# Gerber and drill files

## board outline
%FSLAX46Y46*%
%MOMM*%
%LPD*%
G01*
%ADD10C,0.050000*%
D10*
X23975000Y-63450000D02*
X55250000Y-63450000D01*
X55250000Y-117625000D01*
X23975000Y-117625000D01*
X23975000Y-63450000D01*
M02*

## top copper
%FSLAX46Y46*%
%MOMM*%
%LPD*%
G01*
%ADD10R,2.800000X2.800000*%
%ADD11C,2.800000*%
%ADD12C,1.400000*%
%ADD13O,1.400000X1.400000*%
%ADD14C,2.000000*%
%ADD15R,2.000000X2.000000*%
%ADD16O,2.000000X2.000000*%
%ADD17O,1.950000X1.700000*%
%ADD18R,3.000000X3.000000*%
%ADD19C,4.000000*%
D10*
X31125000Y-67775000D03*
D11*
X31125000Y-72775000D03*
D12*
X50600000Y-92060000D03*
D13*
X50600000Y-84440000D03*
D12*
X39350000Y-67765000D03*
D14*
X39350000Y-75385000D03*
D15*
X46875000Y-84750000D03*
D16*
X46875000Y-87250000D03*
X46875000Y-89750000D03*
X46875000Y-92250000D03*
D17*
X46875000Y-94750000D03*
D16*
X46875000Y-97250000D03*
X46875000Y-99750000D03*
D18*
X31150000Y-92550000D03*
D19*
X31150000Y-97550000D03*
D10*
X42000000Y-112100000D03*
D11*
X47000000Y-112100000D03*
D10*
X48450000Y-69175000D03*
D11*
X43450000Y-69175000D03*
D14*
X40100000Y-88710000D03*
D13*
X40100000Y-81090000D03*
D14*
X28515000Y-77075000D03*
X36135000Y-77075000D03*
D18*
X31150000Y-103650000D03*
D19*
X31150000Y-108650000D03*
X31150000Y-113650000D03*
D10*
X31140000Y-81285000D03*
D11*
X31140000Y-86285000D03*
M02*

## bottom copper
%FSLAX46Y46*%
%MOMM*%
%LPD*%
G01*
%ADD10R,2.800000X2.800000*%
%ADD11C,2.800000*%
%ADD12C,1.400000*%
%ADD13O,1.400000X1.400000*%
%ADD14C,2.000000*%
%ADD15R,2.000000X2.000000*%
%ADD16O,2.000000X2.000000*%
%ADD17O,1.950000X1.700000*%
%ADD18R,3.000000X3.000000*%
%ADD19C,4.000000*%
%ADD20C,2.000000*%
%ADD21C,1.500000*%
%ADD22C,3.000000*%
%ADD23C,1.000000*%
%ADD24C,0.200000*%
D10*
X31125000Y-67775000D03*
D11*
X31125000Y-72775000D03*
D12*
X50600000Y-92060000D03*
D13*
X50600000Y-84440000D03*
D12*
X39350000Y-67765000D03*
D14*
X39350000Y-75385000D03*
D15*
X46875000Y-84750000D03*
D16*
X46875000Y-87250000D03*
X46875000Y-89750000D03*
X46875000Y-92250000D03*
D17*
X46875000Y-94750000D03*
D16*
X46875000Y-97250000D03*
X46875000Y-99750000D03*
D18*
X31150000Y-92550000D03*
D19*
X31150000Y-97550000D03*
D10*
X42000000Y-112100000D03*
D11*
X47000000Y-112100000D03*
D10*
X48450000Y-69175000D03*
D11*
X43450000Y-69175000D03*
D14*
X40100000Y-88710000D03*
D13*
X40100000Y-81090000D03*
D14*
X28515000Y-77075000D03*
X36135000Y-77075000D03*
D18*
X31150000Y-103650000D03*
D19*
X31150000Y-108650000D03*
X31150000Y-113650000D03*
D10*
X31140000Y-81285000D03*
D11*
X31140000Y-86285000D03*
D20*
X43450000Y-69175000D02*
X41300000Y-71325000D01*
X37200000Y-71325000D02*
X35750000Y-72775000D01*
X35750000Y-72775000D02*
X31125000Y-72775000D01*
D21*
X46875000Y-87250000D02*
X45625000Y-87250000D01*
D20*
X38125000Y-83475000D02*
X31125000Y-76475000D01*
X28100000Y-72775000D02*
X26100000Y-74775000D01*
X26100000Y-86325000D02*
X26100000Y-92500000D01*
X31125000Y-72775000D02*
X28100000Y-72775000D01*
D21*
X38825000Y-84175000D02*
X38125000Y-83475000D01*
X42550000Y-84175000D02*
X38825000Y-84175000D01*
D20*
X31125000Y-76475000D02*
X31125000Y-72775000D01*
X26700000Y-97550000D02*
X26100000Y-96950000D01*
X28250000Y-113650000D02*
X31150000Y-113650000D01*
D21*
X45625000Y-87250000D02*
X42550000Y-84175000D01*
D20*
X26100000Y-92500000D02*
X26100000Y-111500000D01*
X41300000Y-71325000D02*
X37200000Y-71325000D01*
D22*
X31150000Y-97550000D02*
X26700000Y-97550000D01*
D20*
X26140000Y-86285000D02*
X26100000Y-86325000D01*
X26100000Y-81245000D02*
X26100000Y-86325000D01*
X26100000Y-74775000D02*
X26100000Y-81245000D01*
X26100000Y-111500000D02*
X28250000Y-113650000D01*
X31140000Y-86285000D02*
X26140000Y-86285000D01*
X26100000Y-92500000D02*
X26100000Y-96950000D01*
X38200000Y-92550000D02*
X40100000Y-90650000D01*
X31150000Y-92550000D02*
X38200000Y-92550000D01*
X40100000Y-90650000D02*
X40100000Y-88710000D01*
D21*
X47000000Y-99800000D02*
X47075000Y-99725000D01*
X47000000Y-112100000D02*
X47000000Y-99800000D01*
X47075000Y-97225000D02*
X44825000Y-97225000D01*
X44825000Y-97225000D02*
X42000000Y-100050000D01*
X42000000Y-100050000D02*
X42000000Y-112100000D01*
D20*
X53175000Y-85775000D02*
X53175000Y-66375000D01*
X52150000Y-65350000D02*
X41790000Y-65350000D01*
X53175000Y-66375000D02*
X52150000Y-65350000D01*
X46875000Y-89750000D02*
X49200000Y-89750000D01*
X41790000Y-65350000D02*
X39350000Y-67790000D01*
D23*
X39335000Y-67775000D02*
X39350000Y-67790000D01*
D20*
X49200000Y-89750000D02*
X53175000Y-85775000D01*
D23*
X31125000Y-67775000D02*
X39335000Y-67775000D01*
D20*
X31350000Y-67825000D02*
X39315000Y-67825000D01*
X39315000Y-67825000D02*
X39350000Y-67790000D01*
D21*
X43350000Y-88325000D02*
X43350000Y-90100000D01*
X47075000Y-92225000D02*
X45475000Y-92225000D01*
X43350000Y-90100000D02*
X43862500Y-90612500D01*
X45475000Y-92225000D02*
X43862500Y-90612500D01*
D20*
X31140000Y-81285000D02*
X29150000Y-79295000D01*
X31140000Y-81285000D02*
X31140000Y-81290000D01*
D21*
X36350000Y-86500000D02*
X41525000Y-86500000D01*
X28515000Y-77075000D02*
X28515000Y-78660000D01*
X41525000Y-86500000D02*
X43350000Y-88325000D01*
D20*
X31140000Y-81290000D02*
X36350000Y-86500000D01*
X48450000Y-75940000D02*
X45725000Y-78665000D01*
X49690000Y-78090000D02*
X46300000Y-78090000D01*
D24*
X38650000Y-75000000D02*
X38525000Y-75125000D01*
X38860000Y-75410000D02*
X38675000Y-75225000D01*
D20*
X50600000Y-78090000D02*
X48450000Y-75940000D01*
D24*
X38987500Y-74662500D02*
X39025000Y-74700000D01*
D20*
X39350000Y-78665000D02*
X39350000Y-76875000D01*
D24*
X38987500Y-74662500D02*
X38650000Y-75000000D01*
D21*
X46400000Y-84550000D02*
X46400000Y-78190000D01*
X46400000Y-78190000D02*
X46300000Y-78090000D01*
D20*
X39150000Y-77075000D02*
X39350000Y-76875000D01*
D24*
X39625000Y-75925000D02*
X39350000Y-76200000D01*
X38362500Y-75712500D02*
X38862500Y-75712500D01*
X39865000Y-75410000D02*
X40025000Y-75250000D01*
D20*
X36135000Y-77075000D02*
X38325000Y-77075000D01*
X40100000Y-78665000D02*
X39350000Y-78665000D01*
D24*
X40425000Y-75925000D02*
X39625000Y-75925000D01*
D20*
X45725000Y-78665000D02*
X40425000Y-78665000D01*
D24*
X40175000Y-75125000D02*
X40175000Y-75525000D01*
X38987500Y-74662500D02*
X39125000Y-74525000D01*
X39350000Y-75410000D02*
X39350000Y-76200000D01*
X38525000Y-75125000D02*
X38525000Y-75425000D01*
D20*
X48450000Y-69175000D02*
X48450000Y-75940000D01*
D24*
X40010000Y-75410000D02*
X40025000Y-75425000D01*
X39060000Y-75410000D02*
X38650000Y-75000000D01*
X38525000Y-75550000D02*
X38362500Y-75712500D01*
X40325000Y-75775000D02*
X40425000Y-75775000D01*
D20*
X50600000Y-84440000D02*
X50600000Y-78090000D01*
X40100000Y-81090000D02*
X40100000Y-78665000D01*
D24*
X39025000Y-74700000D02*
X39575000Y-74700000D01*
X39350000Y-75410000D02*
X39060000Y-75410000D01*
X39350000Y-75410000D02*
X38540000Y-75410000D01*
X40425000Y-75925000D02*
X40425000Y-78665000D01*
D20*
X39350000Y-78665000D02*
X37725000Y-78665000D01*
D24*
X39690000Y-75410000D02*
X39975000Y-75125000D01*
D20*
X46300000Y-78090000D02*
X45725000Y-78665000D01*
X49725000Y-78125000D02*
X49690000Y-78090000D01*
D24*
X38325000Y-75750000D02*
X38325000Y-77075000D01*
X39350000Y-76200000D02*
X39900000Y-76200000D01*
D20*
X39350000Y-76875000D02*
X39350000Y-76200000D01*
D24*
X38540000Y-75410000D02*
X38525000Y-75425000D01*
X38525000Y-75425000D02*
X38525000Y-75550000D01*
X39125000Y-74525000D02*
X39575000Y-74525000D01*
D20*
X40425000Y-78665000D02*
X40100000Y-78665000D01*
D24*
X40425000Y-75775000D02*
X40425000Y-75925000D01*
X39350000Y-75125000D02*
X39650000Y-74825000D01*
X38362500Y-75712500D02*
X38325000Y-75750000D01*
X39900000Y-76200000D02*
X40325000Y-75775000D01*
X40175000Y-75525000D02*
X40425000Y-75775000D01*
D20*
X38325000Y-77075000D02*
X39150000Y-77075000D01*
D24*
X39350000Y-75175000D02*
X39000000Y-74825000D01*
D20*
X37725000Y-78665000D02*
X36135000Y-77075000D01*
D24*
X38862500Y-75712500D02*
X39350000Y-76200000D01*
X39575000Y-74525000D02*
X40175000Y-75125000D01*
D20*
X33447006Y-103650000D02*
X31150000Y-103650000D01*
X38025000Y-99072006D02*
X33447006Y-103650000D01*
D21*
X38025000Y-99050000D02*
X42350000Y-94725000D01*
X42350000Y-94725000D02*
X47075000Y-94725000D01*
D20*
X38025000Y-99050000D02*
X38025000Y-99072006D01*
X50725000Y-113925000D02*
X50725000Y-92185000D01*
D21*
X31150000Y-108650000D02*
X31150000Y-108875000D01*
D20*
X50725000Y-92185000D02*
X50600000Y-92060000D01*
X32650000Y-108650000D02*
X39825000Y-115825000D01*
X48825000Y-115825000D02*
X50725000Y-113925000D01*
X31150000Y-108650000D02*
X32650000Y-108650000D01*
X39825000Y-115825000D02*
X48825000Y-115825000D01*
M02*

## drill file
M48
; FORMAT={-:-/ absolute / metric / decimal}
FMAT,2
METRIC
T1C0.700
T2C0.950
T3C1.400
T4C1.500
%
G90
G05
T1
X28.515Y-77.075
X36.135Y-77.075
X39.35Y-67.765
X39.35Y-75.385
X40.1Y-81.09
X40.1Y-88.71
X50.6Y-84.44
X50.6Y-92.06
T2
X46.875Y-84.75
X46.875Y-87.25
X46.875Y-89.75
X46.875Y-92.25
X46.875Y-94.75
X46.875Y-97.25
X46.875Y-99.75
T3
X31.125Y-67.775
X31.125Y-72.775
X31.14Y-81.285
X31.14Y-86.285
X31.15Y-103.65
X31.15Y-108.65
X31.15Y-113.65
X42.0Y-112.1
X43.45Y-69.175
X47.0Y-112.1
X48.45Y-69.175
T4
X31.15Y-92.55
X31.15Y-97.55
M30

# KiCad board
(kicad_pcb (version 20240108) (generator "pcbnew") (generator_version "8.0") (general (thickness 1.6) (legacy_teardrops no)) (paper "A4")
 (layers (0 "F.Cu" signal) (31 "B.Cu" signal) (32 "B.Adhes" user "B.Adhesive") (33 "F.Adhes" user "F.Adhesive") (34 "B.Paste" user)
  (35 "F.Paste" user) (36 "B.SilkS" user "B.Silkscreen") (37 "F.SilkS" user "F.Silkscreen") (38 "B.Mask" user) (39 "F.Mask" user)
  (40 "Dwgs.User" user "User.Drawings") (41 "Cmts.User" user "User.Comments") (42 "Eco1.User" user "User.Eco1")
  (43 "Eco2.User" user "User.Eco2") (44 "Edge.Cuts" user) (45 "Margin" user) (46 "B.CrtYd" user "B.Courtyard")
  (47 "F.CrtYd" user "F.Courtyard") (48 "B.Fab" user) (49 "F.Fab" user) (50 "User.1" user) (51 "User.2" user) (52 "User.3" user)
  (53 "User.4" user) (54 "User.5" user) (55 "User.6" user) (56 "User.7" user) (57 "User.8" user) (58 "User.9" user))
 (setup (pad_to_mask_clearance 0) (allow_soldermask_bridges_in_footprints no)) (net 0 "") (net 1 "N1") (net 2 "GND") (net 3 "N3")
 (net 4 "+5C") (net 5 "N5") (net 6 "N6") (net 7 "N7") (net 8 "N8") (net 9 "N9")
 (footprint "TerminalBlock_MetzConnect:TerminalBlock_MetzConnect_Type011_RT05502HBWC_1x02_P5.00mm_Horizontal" (layer "F.Cu")
  (at 31.125 67.775 -90)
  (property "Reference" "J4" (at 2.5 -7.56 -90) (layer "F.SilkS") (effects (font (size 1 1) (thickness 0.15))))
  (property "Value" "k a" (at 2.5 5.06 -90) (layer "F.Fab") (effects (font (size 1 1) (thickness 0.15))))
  (pad "1" thru_hole rect (at 0 0 270) (size 2.8 2.8) (drill 1.4) (layers "*.Cu" "*.Mask") (remove_unused_layers no) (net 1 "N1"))
  (pad "2" thru_hole circle (at 5 0 270) (size 2.8 2.8) (drill 1.4) (layers "*.Cu" "*.Mask") (remove_unused_layers no) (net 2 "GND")))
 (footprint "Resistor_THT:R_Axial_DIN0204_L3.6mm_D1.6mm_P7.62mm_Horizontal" (layer "F.Cu") (at 50.6 92.06 90)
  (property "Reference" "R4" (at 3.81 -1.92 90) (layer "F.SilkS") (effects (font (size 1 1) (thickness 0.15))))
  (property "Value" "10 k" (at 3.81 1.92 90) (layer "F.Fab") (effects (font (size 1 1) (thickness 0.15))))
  (pad "1" thru_hole circle (at 0 0 90) (size 1.4 1.4) (drill 0.7) (layers "*.Cu" "*.Mask") (remove_unused_layers no) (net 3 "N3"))
  (pad "2" thru_hole oval (at 7.62 0 90) (size 1.4 1.4) (drill 0.7) (layers "*.Cu" "*.Mask") (remove_unused_layers no) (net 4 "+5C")))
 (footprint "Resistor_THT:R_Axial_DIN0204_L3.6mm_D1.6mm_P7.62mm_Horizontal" (layer "F.Cu") (at 39.35 67.765 -90)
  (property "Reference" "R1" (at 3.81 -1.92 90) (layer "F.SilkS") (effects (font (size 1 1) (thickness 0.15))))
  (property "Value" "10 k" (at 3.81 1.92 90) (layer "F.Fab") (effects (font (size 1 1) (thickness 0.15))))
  (pad "1" thru_hole circle (at 0 0 270) (size 1.4 1.4) (drill 0.7) (layers "*.Cu" "*.Mask") (remove_unused_layers no) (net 1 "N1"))
  (pad "2" thru_hole circle (at 7.62 0 270) (size 2 2) (drill 0.7) (layers "*.Cu" "*.Mask") (remove_unused_layers no) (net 4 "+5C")))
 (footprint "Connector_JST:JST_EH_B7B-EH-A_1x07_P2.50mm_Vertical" (layer "F.Cu") (at 46.875 84.75 -90)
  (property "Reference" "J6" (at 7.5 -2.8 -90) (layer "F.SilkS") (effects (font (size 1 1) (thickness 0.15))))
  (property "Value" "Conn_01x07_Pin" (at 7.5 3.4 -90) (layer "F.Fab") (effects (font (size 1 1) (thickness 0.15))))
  (pad "1" thru_hole rect (at 0 0 270) (size 2 2) (drill 0.95) (layers "*.Cu" "*.Mask") (remove_unused_layers no) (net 4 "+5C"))
  (pad "2" thru_hole oval (at 2.5 0 270) (size 2 2) (drill 0.95) (layers "*.Cu" "*.Mask") (remove_unused_layers no) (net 2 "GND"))
  (pad "3" thru_hole oval (at 5 0 270) (size 2 2) (drill 0.95) (layers "*.Cu" "*.Mask") (remove_unused_layers no) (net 1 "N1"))
  (pad "4" thru_hole oval (at 7.5 0 270) (size 2 2) (drill 0.95) (layers "*.Cu" "*.Mask") (remove_unused_layers no) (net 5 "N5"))
  (pad "5" thru_hole oval (at 10 0 270) (size 1.7 1.95) (drill 0.95) (layers "*.Cu" "*.Mask") (remove_unused_layers no) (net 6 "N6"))
  (pad "6" thru_hole oval (at 12.5 0 270) (size 2 2) (drill 0.95) (layers "*.Cu" "*.Mask") (remove_unused_layers no) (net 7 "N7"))
  (pad "7" thru_hole oval (at 15 0 270) (size 2 2) (drill 0.95) (layers "*.Cu" "*.Mask") (remove_unused_layers no) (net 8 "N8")))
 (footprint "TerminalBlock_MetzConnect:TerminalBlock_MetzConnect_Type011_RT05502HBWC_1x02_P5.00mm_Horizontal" (layer "F.Cu")
  (at 31.15 92.55 -90)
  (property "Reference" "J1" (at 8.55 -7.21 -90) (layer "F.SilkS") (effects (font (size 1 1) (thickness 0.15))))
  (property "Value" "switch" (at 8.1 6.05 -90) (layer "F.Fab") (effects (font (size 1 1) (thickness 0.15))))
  (pad "1" thru_hole rect (at 0 0 270) (size 3 3) (drill 1.5) (layers "*.Cu" "*.Mask") (remove_unused_layers no) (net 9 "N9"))
  (pad "2" thru_hole circle (at 5 0 270) (size 4 4) (drill 1.5) (layers "*.Cu" "*.Mask") (remove_unused_layers no) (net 2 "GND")))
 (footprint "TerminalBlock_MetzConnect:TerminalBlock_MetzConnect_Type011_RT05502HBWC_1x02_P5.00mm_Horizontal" (layer "F.Cu") (at 42 112.1)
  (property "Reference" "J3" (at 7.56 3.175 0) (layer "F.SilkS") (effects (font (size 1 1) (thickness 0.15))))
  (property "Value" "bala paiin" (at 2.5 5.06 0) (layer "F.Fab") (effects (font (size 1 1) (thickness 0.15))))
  (pad "1" thru_hole rect (at 0 0) (size 2.8 2.8) (drill 1.4) (layers "*.Cu" "*.Mask") (remove_unused_layers no) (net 7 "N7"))
  (pad "2" thru_hole circle (at 5 0) (size 2.8 2.8) (drill 1.4) (layers "*.Cu" "*.Mask") (remove_unused_layers no) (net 8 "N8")))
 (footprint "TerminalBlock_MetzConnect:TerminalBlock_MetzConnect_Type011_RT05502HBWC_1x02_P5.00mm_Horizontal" (layer "F.Cu")
  (at 48.45 69.175 180)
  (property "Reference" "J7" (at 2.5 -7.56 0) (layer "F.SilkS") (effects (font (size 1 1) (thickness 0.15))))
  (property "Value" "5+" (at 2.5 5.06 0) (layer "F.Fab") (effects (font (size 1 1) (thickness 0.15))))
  (pad "1" thru_hole rect (at 0 0 180) (size 2.8 2.8) (drill 1.4) (layers "*.Cu" "*.Mask") (remove_unused_layers no) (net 4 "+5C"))
  (pad "2" thru_hole circle (at 5 0 180) (size 2.8 2.8) (drill 1.4) (layers "*.Cu" "*.Mask") (remove_unused_layers no) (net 2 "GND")))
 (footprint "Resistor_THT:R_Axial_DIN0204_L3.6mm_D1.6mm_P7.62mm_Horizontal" (layer "F.Cu") (at 40.1 88.71 90)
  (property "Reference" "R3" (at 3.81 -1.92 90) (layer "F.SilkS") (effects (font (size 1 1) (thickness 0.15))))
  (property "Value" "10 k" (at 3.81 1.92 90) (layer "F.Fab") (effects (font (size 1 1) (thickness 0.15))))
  (pad "1" thru_hole circle (at 0 0 90) (size 2 2) (drill 0.7) (layers "*.Cu" "*.Mask") (remove_unused_layers no) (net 9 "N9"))
  (pad "2" thru_hole oval (at 7.62 0 90) (size 1.4 1.4) (drill 0.7) (layers "*.Cu" "*.Mask") (remove_unused_layers no) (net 4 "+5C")))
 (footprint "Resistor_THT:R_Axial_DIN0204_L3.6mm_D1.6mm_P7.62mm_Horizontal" (layer "F.Cu") (at 28.515 77.075)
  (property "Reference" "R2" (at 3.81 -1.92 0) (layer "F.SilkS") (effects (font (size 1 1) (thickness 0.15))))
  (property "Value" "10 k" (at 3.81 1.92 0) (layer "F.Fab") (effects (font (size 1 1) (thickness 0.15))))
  (pad "1" thru_hole circle (at 0 0) (size 2 2) (drill 0.7) (layers "*.Cu" "*.Mask") (remove_unused_layers no) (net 5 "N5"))
  (pad "2" thru_hole circle (at 7.62 0) (size 2 2) (drill 0.7) (layers "*.Cu" "*.Mask") (remove_unused_layers no) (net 4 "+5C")))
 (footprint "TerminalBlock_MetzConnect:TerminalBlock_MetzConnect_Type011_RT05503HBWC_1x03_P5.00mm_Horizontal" (layer "F.Cu")
  (at 31.15 103.65 -90)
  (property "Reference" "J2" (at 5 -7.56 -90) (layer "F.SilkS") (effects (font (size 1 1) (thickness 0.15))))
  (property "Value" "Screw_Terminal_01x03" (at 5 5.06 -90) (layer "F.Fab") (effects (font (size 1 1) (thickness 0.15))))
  (pad "1" thru_hole rect (at 0 0 270) (size 3 3) (drill 1.4) (layers "*.Cu" "*.Mask") (remove_unused_layers no) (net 6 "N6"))
  (pad "2" thru_hole circle (at 5 0 270) (size 4 4) (drill 1.4) (layers "*.Cu" "*.Mask") (remove_unused_layers no) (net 3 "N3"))
  (pad "3" thru_hole circle (at 10 0 270) (size 4 4) (drill 1.4) (layers "*.Cu" "*.Mask") (remove_unused_layers no) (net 2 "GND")))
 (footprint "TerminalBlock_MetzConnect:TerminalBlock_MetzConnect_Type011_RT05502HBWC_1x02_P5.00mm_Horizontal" (layer "F.Cu")
  (at 31.14 81.285 -90)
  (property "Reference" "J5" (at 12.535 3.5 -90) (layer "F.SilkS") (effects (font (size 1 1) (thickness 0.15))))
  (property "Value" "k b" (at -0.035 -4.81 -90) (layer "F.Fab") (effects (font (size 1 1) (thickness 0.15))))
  (pad "1" thru_hole rect (at 0 0 270) (size 2.8 2.8) (drill 1.4) (layers "*.Cu" "*.Mask") (remove_unused_layers no) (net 5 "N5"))
  (pad "2" thru_hole circle (at 5 0 270) (size 2.8 2.8) (drill 1.4) (layers "*.Cu" "*.Mask") (remove_unused_layers no) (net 2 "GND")))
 (gr_rect (start 23.975 63.45) (end 55.25 117.625) (stroke (width 0.05) (type default)) (fill none) (layer "Edge.Cuts"))
 (segment (start 43.45 69.175) (end 41.3 71.325) (width 2) (layer "B.Cu") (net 2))
 (segment (start 37.2 71.325) (end 35.75 72.775) (width 2) (layer "B.Cu") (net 2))
 (segment (start 35.75 72.775) (end 31.125 72.775) (width 2) (layer "B.Cu") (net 2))
 (segment (start 46.875 87.25) (end 45.625 87.25) (width 1.5) (layer "B.Cu") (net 2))
 (segment (start 38.125 83.475) (end 31.125 76.475) (width 2) (layer "B.Cu") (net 2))
 (segment (start 28.1 72.775) (end 26.1 74.775) (width 2) (layer "B.Cu") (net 2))
 (segment (start 26.1 86.325) (end 26.1 92.5) (width 2) (layer "B.Cu") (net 2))
 (segment (start 31.125 72.775) (end 28.1 72.775) (width 2) (layer "B.Cu") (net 2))
 (segment (start 38.825 84.175) (end 38.125 83.475) (width 1.5) (layer "B.Cu") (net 2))
 (segment (start 42.55 84.175) (end 38.825 84.175) (width 1.5) (layer "B.Cu") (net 2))
 (segment (start 31.125 76.475) (end 31.125 72.775) (width 2) (layer "B.Cu") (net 2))
 (segment (start 26.7 97.55) (end 26.1 96.95) (width 2) (layer "B.Cu") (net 2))
 (segment (start 28.25 113.65) (end 31.15 113.65) (width 2) (layer "B.Cu") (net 2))
 (segment (start 45.625 87.25) (end 42.55 84.175) (width 1.5) (layer "B.Cu") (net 2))
 (segment (start 26.1 92.5) (end 26.1 111.5) (width 2) (layer "B.Cu") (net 2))
 (segment (start 41.3 71.325) (end 37.2 71.325) (width 2) (layer "B.Cu") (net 2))
 (segment (start 31.15 97.55) (end 26.7 97.55) (width 3) (layer "B.Cu") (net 2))
 (segment (start 26.14 86.285) (end 26.1 86.325) (width 2) (layer "B.Cu") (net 2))
 (segment (start 26.1 81.245) (end 26.1 86.325) (width 2) (layer "B.Cu") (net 2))
 (segment (start 26.1 74.775) (end 26.1 81.245) (width 2) (layer "B.Cu") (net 2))
 (segment (start 26.1 111.5) (end 28.25 113.65) (width 2) (layer "B.Cu") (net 2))
 (segment (start 31.14 86.285) (end 26.14 86.285) (width 2) (layer "B.Cu") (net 2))
 (segment (start 26.1 92.5) (end 26.1 96.95) (width 2) (layer "B.Cu") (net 2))
 (segment (start 38.2 92.55) (end 40.1 90.65) (width 2) (layer "B.Cu") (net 9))
 (segment (start 31.15 92.55) (end 38.2 92.55) (width 2) (layer "B.Cu") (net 9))
 (segment (start 40.1 90.65) (end 40.1 88.71) (width 2) (layer "B.Cu") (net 9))
 (segment (start 47 99.8) (end 47.075 99.725) (width 1.5) (layer "B.Cu") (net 8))
 (segment (start 47 112.1) (end 47 99.8) (width 1.5) (layer "B.Cu") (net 8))
 (segment (start 47.075 97.225) (end 44.825 97.225) (width 1.5) (layer "B.Cu") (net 7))
 (segment (start 44.825 97.225) (end 42 100.05) (width 1.5) (layer "B.Cu") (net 7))
 (segment (start 42 100.05) (end 42 112.1) (width 1.5) (layer "B.Cu") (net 7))
 (segment (start 53.175 85.775) (end 53.175 66.375) (width 2) (layer "B.Cu") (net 1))
 (segment (start 52.15 65.35) (end 41.79 65.35) (width 2) (layer "B.Cu") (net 1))
 (segment (start 53.175 66.375) (end 52.15 65.35) (width 2) (layer "B.Cu") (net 1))
 (segment (start 46.875 89.75) (end 49.2 89.75) (width 2) (layer "B.Cu") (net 1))
 (segment (start 41.79 65.35) (end 39.35 67.79) (width 2) (layer "B.Cu") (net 1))
 (segment (start 39.335 67.775) (end 39.35 67.79) (width 1) (layer "B.Cu") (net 1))
 (segment (start 49.2 89.75) (end 53.175 85.775) (width 2) (layer "B.Cu") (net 1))
 (segment (start 31.125 67.775) (end 39.335 67.775) (width 1) (layer "B.Cu") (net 1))
 (segment (start 31.35 67.825) (end 39.315 67.825) (width 2) (layer "B.Cu") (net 1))
 (segment (start 39.315 67.825) (end 39.35 67.79) (width 2) (layer "B.Cu") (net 1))
 (segment (start 43.35 88.325) (end 43.35 90.1) (width 1.5) (layer "B.Cu") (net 5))
 (segment (start 47.075 92.225) (end 45.475 92.225) (width 1.5) (layer "B.Cu") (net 5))
 (segment (start 43.35 90.1) (end 43.8625 90.6125) (width 1.5) (layer "B.Cu") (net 5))
 (segment (start 45.475 92.225) (end 43.8625 90.6125) (width 1.5) (layer "B.Cu") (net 5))
 (segment (start 31.14 81.285) (end 29.15 79.295) (width 2) (layer "B.Cu") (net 5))
 (segment (start 31.14 81.285) (end 31.14 81.29) (width 2) (layer "B.Cu") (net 5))
 (segment (start 36.35 86.5) (end 41.525 86.5) (width 1.5) (layer "B.Cu") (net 5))
 (segment (start 28.515 77.075) (end 28.515 78.66) (width 1.5) (layer "B.Cu") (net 5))
 (segment (start 41.525 86.5) (end 43.35 88.325) (width 1.5) (layer "B.Cu") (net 5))
 (segment (start 31.14 81.29) (end 36.35 86.5) (width 2) (layer "B.Cu") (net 5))
 (segment (start 48.45 75.94) (end 45.725 78.665) (width 2) (layer "B.Cu") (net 4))
 (segment (start 49.69 78.09) (end 46.3 78.09) (width 2) (layer "B.Cu") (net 4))
 (segment (start 38.65 75) (end 38.525 75.125) (width 0.2) (layer "B.Cu") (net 4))
 (segment (start 38.86 75.41) (end 38.675 75.225) (width 0.2) (layer "B.Cu") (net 4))
 (segment (start 50.6 78.09) (end 48.45 75.94) (width 2) (layer "B.Cu") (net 4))
 (segment (start 38.9875 74.6625) (end 39.025 74.7) (width 0.2) (layer "B.Cu") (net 4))
 (segment (start 39.35 78.665) (end 39.35 76.875) (width 2) (layer "B.Cu") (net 4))
 (segment (start 38.9875 74.6625) (end 38.65 75) (width 0.2) (layer "B.Cu") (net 4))
 (segment (start 46.4 84.55) (end 46.4 78.19) (width 1.5) (layer "B.Cu") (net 4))
 (segment (start 46.4 78.19) (end 46.3 78.09) (width 1.5) (layer "B.Cu") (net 4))
 (segment (start 39.15 77.075) (end 39.35 76.875) (width 2) (layer "B.Cu") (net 4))
 (segment (start 39.625 75.925) (end 39.35 76.2) (width 0.2) (layer "B.Cu") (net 4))
 (segment (start 38.3625 75.7125) (end 38.8625 75.7125) (width 0.2) (layer "B.Cu") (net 4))
 (segment (start 39.865 75.41) (end 40.025 75.25) (width 0.2) (layer "B.Cu") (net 4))
 (segment (start 36.135 77.075) (end 38.325 77.075) (width 2) (layer "B.Cu") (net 4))
 (segment (start 40.1 78.665) (end 39.35 78.665) (width 2) (layer "B.Cu") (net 4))
 (segment (start 40.425 75.925) (end 39.625 75.925) (width 0.2) (layer "B.Cu") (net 4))
 (segment (start 45.725 78.665) (end 40.425 78.665) (width 2) (layer "B.Cu") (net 4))
 (segment (start 40.175 75.125) (end 40.175 75.525) (width 0.2) (layer "B.Cu") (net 4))
 (segment (start 38.9875 74.6625) (end 39.125 74.525) (width 0.2) (layer "B.Cu") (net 4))
 (segment (start 39.35 75.41) (end 39.35 76.2) (width 0.2) (layer "B.Cu") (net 4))
 (segment (start 38.525 75.125) (end 38.525 75.425) (width 0.2) (layer "B.Cu") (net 4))
 (segment (start 48.45 69.175) (end 48.45 75.94) (width 2) (layer "B.Cu") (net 4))
 (segment (start 40.01 75.41) (end 40.025 75.425) (width 0.2) (layer "B.Cu") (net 4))
 (segment (start 39.06 75.41) (end 38.65 75) (width 0.2) (layer "B.Cu") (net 4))
 (segment (start 38.525 75.55) (end 38.3625 75.7125) (width 0.2) (layer "B.Cu") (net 4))
 (segment (start 40.325 75.775) (end 40.425 75.775) (width 0.2) (layer "B.Cu") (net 4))
 (segment (start 50.6 84.44) (end 50.6 78.09) (width 2) (layer "B.Cu") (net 4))
 (segment (start 40.1 81.09) (end 40.1 78.665) (width 2) (layer "B.Cu") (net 4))
 (segment (start 39.025 74.7) (end 39.575 74.7) (width 0.2) (layer "B.Cu") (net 4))
 (segment (start 39.35 75.41) (end 39.06 75.41) (width 0.2) (layer "B.Cu") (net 4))
 (segment (start 39.35 75.41) (end 38.54 75.41) (width 0.2) (layer "B.Cu") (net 4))
 (segment (start 40.425 75.925) (end 40.425 78.665) (width 0.2) (layer "B.Cu") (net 4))
 (segment (start 39.35 78.665) (end 37.725 78.665) (width 2) (layer "B.Cu") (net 4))
 (segment (start 39.69 75.41) (end 39.975 75.125) (width 0.2) (layer "B.Cu") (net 4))
 (segment (start 46.3 78.09) (end 45.725 78.665) (width 2) (layer "B.Cu") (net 4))
 (segment (start 49.725 78.125) (end 49.69 78.09) (width 2) (layer "B.Cu") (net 4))
 (segment (start 38.325 75.75) (end 38.325 77.075) (width 0.2) (layer "B.Cu") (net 4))
 (segment (start 39.35 76.2) (end 39.9 76.2) (width 0.2) (layer "B.Cu") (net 4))
 (segment (start 39.35 76.875) (end 39.35 76.2) (width 2) (layer "B.Cu") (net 4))
 (segment (start 38.54 75.41) (end 38.525 75.425) (width 0.2) (layer "B.Cu") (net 4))
 (segment (start 38.525 75.425) (end 38.525 75.55) (width 0.2) (layer "B.Cu") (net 4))
 (segment (start 39.125 74.525) (end 39.575 74.525) (width 0.2) (layer "B.Cu") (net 4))
 (segment (start 40.425 78.665) (end 40.1 78.665) (width 2) (layer "B.Cu") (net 4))
 (segment (start 40.425 75.775) (end 40.425 75.925) (width 0.2) (layer "B.Cu") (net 4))
 (segment (start 39.35 75.125) (end 39.65 74.825) (width 0.2) (layer "B.Cu") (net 4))
 (segment (start 38.3625 75.7125) (end 38.325 75.75) (width 0.2) (layer "B.Cu") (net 4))
 (segment (start 39.9 76.2) (end 40.325 75.775) (width 0.2) (layer "B.Cu") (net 4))
 (segment (start 40.175 75.525) (end 40.425 75.775) (width 0.2) (layer "B.Cu") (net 4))
 (segment (start 38.325 77.075) (end 39.15 77.075) (width 2) (layer "B.Cu") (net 4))
 (segment (start 39.35 75.175) (end 39 74.825) (width 0.2) (layer "B.Cu") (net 4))
 (segment (start 37.725 78.665) (end 36.135 77.075) (width 2) (layer "B.Cu") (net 4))
 (segment (start 38.8625 75.7125) (end 39.35 76.2) (width 0.2) (layer "B.Cu") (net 4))
 (segment (start 39.575 74.525) (end 40.175 75.125) (width 0.2) (layer "B.Cu") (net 4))
 (segment (start 33.447006 103.65) (end 31.15 103.65) (width 2) (layer "B.Cu") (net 6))
 (segment (start 38.025 99.072006) (end 33.447006 103.65) (width 2) (layer "B.Cu") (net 6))
 (segment (start 38.025 99.05) (end 42.35 94.725) (width 1.5) (layer "B.Cu") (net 6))
 (segment (start 42.35 94.725) (end 47.075 94.725) (width 1.5) (layer "B.Cu") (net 6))
 (segment (start 38.025 99.05) (end 38.025 99.072006) (width 2) (layer "B.Cu") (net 6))
 (segment (start 50.725 113.925) (end 50.725 92.185) (width 2) (layer "B.Cu") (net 3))
 (segment (start 31.15 108.65) (end 31.15 108.875) (width 1.5) (layer "B.Cu") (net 3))
 (segment (start 50.725 92.185) (end 50.6 92.06) (width 2) (layer "B.Cu") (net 3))
 (segment (start 32.65 108.65) (end 39.825 115.825) (width 2) (layer "B.Cu") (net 3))
 (segment (start 48.825 115.825) (end 50.725 113.925) (width 2) (layer "B.Cu") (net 3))
 (segment (start 31.15 108.65) (end 32.65 108.65) (width 2) (layer "B.Cu") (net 3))
 (segment (start 39.825 115.825) (end 48.825 115.825) (width 2) (layer "B.Cu") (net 3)))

